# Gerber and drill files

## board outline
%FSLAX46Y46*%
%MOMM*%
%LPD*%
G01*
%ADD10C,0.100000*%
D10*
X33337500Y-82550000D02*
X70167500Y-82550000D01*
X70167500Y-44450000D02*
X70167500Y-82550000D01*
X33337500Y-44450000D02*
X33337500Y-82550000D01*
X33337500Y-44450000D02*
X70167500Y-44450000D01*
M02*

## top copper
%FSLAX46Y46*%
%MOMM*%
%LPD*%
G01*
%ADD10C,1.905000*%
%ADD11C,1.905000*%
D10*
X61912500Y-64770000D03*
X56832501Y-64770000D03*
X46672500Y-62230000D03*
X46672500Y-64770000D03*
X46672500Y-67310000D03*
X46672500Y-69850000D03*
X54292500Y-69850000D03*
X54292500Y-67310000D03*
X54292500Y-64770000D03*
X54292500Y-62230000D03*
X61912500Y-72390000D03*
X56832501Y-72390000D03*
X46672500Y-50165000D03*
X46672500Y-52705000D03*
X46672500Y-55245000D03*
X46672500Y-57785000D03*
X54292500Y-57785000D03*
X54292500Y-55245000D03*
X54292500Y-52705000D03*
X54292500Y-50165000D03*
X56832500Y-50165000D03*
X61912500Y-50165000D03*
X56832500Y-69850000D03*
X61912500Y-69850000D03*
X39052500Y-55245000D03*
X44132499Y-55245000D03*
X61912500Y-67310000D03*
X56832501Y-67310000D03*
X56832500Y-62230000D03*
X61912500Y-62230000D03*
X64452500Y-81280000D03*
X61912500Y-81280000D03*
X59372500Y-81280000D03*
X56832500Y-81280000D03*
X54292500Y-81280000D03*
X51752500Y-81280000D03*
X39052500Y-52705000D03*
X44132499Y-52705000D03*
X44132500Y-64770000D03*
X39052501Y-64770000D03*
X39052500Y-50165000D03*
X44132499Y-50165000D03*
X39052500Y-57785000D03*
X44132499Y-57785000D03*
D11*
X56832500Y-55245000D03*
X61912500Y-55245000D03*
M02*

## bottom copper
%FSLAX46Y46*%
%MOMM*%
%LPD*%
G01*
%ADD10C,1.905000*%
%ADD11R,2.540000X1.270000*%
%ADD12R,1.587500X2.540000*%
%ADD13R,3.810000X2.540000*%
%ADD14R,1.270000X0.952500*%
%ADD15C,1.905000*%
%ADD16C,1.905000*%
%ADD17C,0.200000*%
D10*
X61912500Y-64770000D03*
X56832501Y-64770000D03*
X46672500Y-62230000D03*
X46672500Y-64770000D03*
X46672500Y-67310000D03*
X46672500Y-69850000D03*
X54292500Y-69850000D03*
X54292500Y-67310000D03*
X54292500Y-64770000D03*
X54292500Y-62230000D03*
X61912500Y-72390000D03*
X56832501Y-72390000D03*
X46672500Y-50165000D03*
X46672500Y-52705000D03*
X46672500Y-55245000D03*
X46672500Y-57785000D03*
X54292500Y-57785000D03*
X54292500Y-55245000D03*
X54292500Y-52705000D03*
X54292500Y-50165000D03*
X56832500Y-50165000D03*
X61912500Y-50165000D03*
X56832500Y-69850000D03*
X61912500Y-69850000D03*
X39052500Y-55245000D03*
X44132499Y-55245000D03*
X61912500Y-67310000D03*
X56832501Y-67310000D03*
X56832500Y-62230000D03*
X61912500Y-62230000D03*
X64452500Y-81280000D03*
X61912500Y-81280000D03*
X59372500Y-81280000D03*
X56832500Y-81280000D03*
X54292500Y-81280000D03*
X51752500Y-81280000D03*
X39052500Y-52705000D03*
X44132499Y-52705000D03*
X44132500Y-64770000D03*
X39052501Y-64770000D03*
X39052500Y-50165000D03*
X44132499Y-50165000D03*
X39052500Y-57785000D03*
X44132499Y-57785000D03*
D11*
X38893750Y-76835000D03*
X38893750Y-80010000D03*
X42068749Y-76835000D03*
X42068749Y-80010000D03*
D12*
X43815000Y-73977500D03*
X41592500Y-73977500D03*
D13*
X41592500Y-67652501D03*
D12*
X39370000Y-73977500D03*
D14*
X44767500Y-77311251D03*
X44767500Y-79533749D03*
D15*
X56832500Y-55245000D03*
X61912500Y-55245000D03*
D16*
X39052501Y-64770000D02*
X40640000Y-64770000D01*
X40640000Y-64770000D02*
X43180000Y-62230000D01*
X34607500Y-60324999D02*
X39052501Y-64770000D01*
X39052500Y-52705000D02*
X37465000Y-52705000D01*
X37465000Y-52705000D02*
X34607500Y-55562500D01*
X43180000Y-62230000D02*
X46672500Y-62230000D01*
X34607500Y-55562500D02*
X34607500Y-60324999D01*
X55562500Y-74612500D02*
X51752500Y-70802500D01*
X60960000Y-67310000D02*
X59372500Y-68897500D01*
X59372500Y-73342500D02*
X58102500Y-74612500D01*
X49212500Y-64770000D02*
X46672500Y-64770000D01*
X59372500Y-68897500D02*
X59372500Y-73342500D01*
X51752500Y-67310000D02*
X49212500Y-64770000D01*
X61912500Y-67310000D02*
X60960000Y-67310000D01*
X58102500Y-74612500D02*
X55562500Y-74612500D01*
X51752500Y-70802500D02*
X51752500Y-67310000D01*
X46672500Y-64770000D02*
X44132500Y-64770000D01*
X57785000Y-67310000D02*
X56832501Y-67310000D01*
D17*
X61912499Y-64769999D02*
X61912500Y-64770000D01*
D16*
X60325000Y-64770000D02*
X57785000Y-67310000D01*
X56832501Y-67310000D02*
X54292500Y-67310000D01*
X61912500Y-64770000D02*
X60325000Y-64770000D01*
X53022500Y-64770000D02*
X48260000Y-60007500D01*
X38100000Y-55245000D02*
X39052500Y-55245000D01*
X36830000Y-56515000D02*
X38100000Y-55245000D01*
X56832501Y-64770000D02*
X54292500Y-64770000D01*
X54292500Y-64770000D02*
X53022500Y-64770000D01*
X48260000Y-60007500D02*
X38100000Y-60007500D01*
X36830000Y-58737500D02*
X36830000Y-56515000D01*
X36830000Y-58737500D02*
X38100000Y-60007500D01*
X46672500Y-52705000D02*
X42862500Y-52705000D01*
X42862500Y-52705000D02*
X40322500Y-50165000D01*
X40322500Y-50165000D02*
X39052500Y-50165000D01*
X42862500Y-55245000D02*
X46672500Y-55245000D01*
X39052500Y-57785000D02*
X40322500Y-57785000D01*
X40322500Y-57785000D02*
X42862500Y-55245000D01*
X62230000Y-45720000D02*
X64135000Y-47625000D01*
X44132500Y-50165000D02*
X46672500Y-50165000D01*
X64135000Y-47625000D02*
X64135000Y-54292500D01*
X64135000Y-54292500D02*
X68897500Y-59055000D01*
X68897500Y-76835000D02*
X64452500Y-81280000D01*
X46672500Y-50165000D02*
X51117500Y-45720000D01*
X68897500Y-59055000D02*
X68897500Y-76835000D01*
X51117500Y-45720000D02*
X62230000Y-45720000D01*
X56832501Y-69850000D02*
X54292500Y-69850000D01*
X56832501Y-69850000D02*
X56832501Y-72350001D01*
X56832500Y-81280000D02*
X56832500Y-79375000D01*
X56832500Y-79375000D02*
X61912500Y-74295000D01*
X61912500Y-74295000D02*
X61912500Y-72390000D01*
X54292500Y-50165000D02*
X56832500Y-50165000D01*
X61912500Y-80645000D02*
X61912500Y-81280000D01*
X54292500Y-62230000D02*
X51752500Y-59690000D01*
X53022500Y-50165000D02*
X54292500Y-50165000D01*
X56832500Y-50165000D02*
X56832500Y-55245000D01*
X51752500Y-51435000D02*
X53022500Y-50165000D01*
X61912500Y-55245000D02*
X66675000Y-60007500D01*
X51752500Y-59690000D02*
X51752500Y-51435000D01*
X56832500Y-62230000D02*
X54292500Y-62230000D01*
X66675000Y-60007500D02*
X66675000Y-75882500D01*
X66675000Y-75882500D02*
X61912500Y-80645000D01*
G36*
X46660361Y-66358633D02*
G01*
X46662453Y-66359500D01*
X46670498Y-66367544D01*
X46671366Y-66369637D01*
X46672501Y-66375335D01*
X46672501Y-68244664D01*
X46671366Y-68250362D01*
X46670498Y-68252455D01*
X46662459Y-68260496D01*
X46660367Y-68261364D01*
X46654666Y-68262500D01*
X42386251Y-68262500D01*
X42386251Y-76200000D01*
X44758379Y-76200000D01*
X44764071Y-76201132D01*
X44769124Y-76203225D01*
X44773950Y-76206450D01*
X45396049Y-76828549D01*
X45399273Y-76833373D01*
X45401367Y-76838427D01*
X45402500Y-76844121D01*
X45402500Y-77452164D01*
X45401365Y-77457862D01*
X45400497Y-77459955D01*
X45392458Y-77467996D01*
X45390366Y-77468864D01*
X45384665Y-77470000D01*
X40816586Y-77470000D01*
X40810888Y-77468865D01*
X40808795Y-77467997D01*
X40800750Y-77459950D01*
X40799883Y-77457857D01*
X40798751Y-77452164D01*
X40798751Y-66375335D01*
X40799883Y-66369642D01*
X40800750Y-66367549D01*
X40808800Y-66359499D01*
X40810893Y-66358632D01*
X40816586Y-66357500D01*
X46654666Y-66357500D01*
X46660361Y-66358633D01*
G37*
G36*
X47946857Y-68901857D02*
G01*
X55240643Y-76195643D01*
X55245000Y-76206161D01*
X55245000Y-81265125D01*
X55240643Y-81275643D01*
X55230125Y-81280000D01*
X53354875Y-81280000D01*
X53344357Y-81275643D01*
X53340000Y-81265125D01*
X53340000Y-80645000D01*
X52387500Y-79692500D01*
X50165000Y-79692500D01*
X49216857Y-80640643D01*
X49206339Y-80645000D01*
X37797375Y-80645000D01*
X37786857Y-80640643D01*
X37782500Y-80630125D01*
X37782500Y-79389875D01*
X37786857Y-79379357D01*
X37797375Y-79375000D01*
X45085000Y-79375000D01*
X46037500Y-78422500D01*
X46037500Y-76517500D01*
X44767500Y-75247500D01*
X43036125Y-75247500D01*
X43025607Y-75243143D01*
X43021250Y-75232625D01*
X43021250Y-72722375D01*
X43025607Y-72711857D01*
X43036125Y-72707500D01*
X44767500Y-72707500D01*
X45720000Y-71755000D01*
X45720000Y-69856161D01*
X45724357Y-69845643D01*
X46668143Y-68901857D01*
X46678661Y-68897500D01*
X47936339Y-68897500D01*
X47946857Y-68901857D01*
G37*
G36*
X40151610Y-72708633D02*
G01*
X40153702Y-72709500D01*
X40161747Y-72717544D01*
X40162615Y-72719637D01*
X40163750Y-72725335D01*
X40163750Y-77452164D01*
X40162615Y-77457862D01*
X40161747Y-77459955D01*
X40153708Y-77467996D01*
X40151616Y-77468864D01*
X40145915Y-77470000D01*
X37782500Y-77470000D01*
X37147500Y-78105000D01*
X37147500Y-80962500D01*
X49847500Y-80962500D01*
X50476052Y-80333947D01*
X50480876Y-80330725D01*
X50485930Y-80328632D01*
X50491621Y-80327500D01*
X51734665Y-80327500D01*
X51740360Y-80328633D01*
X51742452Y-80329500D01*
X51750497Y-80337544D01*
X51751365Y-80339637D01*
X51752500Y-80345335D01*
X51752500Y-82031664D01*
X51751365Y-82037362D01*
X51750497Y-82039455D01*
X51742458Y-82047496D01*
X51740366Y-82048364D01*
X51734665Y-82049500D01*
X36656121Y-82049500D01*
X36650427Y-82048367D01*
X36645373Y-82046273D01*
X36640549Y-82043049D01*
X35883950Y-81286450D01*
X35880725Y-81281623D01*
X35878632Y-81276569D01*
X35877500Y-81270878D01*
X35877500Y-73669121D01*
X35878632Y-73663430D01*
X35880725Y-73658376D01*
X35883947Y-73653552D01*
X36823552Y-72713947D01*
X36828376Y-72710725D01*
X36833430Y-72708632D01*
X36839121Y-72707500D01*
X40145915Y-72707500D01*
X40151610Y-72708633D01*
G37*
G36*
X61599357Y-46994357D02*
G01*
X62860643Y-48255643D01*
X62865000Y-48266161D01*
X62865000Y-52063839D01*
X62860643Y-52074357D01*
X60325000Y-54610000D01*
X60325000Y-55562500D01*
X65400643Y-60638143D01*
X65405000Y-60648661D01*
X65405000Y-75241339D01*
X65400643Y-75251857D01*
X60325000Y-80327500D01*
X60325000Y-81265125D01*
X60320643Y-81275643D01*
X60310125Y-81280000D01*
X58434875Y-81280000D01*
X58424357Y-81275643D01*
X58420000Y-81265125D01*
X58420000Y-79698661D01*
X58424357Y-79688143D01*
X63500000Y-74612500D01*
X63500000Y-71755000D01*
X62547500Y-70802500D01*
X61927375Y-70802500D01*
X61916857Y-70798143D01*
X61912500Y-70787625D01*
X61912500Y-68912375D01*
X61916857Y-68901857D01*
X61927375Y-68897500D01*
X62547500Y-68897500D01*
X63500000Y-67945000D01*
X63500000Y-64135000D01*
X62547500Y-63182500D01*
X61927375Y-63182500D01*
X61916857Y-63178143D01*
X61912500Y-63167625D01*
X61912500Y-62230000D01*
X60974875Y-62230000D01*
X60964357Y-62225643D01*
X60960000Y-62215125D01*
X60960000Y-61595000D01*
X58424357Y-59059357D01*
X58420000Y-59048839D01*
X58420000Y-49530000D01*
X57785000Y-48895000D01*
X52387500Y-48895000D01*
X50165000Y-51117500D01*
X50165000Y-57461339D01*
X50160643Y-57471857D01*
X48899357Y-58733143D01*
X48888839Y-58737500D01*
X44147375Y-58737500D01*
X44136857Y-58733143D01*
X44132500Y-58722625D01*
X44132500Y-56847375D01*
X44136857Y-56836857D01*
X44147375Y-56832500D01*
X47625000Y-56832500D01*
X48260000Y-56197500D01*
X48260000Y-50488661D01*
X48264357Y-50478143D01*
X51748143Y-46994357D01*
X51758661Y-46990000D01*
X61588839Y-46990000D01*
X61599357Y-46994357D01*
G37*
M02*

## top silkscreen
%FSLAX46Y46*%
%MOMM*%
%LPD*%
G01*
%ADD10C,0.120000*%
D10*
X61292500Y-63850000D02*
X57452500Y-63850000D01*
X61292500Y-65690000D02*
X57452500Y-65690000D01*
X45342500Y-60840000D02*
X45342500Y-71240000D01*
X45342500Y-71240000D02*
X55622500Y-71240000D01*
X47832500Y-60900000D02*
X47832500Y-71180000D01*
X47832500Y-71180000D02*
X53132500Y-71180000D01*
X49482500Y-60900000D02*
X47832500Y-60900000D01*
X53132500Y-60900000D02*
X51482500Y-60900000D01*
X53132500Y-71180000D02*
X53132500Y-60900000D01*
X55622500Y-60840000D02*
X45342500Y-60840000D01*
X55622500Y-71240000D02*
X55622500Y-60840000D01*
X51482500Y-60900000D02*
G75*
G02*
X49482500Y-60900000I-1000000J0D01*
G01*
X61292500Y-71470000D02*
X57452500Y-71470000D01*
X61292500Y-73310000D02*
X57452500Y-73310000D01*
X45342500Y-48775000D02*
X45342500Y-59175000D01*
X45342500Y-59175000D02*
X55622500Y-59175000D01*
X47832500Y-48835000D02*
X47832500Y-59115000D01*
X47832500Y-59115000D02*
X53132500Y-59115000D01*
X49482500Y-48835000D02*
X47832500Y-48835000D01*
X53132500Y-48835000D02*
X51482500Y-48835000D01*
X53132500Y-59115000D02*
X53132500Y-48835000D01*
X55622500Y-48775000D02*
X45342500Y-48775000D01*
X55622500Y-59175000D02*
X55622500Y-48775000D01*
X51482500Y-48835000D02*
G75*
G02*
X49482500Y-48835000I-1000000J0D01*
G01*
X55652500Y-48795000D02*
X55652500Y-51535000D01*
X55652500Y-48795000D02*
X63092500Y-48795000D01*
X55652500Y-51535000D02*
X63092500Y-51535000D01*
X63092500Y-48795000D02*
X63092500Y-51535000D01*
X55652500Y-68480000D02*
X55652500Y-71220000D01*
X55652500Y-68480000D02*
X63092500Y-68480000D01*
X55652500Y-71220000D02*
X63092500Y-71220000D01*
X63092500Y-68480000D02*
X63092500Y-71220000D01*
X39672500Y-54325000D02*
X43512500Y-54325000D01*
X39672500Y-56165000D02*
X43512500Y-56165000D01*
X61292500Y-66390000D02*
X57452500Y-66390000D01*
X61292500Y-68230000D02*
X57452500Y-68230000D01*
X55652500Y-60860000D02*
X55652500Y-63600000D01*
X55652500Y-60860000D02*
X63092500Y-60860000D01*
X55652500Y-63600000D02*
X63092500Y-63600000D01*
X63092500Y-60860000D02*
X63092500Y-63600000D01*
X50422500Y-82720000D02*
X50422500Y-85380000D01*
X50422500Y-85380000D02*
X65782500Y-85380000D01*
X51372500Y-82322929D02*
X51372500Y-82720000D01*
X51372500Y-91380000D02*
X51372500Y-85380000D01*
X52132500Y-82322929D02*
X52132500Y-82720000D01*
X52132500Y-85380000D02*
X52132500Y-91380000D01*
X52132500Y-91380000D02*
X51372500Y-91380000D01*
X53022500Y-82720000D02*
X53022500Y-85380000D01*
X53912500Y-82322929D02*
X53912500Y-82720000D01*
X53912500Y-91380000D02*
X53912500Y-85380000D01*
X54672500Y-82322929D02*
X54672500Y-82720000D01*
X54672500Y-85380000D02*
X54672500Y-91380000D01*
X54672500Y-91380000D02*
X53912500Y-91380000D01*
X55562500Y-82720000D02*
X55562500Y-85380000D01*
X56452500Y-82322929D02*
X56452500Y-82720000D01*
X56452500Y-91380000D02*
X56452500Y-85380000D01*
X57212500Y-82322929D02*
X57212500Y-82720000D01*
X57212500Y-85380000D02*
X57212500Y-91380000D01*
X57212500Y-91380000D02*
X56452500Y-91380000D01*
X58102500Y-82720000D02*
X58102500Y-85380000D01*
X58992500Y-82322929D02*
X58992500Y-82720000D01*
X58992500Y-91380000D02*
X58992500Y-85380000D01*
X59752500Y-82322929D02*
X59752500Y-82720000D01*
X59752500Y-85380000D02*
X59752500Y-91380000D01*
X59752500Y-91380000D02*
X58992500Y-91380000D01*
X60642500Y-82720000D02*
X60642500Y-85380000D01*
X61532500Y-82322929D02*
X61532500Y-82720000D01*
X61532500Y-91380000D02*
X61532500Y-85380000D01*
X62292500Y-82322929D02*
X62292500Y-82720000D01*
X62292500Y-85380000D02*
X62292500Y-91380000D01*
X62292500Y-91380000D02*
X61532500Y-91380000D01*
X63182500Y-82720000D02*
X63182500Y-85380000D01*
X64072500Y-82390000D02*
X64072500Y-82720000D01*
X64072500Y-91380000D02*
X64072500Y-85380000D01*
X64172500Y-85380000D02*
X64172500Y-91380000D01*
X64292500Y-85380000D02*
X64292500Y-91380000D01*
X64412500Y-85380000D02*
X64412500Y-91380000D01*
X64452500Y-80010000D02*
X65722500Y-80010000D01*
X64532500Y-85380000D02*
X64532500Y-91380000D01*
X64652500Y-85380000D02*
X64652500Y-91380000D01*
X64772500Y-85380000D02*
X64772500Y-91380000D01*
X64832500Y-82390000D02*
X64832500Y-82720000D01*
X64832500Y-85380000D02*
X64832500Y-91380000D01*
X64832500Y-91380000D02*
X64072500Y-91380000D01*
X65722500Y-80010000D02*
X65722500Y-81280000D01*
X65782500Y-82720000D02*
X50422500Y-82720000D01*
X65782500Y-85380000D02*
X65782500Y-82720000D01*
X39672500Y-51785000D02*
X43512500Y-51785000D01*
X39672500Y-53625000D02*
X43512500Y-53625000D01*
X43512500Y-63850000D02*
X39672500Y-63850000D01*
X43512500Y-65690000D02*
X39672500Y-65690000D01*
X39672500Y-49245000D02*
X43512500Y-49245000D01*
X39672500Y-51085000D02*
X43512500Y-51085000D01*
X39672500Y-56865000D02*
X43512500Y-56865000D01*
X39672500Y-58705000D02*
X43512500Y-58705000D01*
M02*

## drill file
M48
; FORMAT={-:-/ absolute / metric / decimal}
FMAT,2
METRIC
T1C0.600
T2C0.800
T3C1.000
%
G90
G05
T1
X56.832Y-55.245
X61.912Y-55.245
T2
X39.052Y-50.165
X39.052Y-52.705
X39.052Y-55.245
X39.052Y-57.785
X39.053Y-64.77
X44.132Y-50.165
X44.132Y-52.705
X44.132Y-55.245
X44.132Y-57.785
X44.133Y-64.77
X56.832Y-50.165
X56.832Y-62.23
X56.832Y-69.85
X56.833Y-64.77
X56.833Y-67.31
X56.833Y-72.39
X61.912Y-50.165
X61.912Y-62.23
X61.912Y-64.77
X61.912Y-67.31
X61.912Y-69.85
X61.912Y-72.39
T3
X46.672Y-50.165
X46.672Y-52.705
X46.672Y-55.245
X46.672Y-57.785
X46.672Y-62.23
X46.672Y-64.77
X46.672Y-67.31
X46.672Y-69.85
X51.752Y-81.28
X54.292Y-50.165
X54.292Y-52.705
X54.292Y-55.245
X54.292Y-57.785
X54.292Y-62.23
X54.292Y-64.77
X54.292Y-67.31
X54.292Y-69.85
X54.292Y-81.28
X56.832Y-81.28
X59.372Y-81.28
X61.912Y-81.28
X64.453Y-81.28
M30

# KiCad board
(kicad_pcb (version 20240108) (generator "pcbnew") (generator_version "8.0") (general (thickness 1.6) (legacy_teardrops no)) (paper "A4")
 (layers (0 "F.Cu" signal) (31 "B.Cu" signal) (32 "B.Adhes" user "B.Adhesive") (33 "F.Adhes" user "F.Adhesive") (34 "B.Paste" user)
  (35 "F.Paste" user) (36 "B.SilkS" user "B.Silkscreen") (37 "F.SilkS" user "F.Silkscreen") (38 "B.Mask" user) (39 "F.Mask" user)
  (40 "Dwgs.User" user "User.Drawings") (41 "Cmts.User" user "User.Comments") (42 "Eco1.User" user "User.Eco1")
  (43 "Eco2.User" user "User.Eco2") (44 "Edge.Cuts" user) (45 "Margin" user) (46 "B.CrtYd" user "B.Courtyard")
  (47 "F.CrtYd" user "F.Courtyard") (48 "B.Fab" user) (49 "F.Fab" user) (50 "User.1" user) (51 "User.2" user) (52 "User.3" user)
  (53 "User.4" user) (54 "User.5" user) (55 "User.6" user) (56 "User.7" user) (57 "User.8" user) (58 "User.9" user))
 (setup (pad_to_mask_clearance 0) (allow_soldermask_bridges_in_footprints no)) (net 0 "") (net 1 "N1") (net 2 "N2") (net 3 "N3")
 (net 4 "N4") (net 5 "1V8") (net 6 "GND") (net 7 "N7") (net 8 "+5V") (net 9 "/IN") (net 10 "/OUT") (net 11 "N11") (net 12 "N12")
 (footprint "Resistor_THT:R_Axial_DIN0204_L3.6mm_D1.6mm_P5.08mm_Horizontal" (layer "F.Cu") (at 61.9125 64.77 180)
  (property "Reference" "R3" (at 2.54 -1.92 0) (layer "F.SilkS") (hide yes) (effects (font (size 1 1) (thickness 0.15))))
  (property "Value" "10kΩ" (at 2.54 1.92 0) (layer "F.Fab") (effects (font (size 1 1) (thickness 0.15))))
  (fp_line (start 0.62 0.92) (end 4.46 0.92) (stroke (width 0.12) (type solid)) (layer "F.SilkS"))
  (fp_line (start 0.62 -0.92) (end 4.46 -0.92) (stroke (width 0.12) (type solid)) (layer "F.SilkS"))
  (pad "1" thru_hole circle (at 0 0 180) (size 1.905 1.905) (drill 0.8) (layers "*.Cu" "*.Mask") (remove_unused_layers no) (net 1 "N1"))
  (pad "2" thru_hole circle (at 5.079999 0 180) (size 1.905 1.905) (drill 0.8) (layers "*.Cu" "*.Mask") (remove_unused_layers no)
   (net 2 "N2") (thermal_bridge_angle 90)))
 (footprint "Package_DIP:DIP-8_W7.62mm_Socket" (layer "F.Cu") (at 50.4825 66.04)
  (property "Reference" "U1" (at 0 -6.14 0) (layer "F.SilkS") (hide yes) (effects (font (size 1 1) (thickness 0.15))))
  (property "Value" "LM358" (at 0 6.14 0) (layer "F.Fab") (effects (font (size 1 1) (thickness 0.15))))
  (fp_line (start -5.14 -5.2) (end -5.14 5.2) (stroke (width 0.12) (type solid)) (layer "F.SilkS"))
  (fp_line (start -5.14 5.2) (end 5.14 5.2) (stroke (width 0.12) (type solid)) (layer "F.SilkS"))
  (fp_line (start -2.65 -5.14) (end -2.65 5.14) (stroke (width 0.12) (type solid)) (layer "F.SilkS"))
  (fp_line (start -2.65 5.14) (end 2.65 5.14) (stroke (width 0.12) (type solid)) (layer "F.SilkS"))
  (fp_line (start -1 -5.14) (end -2.65 -5.14) (stroke (width 0.12) (type solid)) (layer "F.SilkS"))
  (fp_line (start 2.65 -5.14) (end 1 -5.14) (stroke (width 0.12) (type solid)) (layer "F.SilkS"))
  (fp_line (start 2.65 5.14) (end 2.65 -5.14) (stroke (width 0.12) (type solid)) (layer "F.SilkS"))
  (fp_line (start 5.14 -5.2) (end -5.14 -5.2) (stroke (width 0.12) (type solid)) (layer "F.SilkS"))
  (fp_line (start 5.14 5.2) (end 5.14 -5.2) (stroke (width 0.12) (type solid)) (layer "F.SilkS"))
  (fp_arc (start 1 -5.14) (mid 0 -4.14) (end -1 -5.14) (stroke (width 0.12) (type solid)) (layer "F.SilkS"))
  (pad "1" thru_hole circle (at -3.81 -3.81) (size 1.905 1.905) (drill 1) (layers "*.Cu" "*.Mask") (remove_unused_layers no) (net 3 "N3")
   (thermal_bridge_angle 90))
  (pad "2" thru_hole circle (at -3.81 -1.27) (size 1.905 1.905) (drill 1) (layers "*.Cu" "*.Mask") (remove_unused_layers no) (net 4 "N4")
   (thermal_bridge_angle 90))
  (pad "3" thru_hole circle (at -3.81 1.27) (size 1.905 1.905) (drill 1) (layers "*.Cu" "*.Mask") (remove_unused_layers no) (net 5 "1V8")
   (thermal_bridge_angle 90))
  (pad "4" thru_hole circle (at -3.81 3.81) (size 1.905 1.905) (drill 1) (layers "*.Cu" "*.Mask") (remove_unused_layers no) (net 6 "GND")
   (thermal_bridge_angle 90))
  (pad "5" thru_hole circle (at 3.81 3.81) (size 1.905 1.905) (drill 1) (layers "*.Cu" "*.Mask") (remove_unused_layers no) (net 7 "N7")
   (thermal_bridge_angle 90))
  (pad "6" thru_hole circle (at 3.81 1.27) (size 1.905 1.905) (drill 1) (layers "*.Cu" "*.Mask") (remove_unused_layers no) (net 1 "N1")
   (thermal_bridge_angle 90))
  (pad "7" thru_hole circle (at 3.81 -1.27) (size 1.905 1.905) (drill 1) (layers "*.Cu" "*.Mask") (remove_unused_layers no) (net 2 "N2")
   (thermal_bridge_angle 90))
  (pad "8" thru_hole circle (at 3.81 -3.81) (size 1.905 1.905) (drill 1) (layers "*.Cu" "*.Mask") (remove_unused_layers no) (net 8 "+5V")
   (thermal_bridge_angle 90)))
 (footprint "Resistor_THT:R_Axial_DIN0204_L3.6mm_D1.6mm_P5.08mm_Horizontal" (layer "F.Cu") (at 61.9125 72.39 180)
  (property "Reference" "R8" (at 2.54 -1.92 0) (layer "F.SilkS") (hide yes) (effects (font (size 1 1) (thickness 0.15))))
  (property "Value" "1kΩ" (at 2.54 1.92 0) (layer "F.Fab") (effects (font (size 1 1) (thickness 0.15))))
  (fp_line (start 0.62 0.92) (end 4.46 0.92) (stroke (width 0.12) (type solid)) (layer "F.SilkS"))
  (fp_line (start 0.62 -0.92) (end 4.46 -0.92) (stroke (width 0.12) (type solid)) (layer "F.SilkS"))
  (pad "1" thru_hole circle (at 0 0 180) (size 1.905 1.905) (drill 0.8) (layers "*.Cu" "*.Mask") (remove_unused_layers no) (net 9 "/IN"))
  (pad "2" thru_hole circle (at 5.079999 0 180) (size 1.905 1.905) (drill 0.8) (layers "*.Cu" "*.Mask") (remove_unused_layers no)
   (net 7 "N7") (thermal_bridge_angle 90)))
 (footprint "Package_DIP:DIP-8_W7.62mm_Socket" (layer "F.Cu") (at 50.4825 53.975)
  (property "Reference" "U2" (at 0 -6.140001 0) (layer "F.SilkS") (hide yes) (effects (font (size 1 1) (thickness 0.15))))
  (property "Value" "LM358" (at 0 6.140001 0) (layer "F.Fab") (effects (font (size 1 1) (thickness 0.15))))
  (fp_line (start -5.14 -5.2) (end -5.14 5.2) (stroke (width 0.12) (type solid)) (layer "F.SilkS"))
  (fp_line (start -5.14 5.2) (end 5.14 5.2) (stroke (width 0.12) (type solid)) (layer "F.SilkS"))
  (fp_line (start -2.65 -5.14) (end -2.65 5.14) (stroke (width 0.12) (type solid)) (layer "F.SilkS"))
  (fp_line (start -2.65 5.14) (end 2.65 5.14) (stroke (width 0.12) (type solid)) (layer "F.SilkS"))
  (fp_line (start -1 -5.14) (end -2.65 -5.14) (stroke (width 0.12) (type solid)) (layer "F.SilkS"))
  (fp_line (start 2.65 -5.14) (end 1 -5.14) (stroke (width 0.12) (type solid)) (layer "F.SilkS"))
  (fp_line (start 2.65 5.14) (end 2.65 -5.14) (stroke (width 0.12) (type solid)) (layer "F.SilkS"))
  (fp_line (start 5.14 -5.2) (end -5.14 -5.2) (stroke (width 0.12) (type solid)) (layer "F.SilkS"))
  (fp_line (start 5.14 5.2) (end 5.14 -5.2) (stroke (width 0.12) (type solid)) (layer "F.SilkS"))
  (fp_arc (start 1 -5.14) (mid 0 -4.14) (end -1 -5.14) (stroke (width 0.12) (type solid)) (layer "F.SilkS"))
  (pad "1" thru_hole circle (at -3.81 -3.81) (size 1.905 1.905) (drill 1) (layers "*.Cu" "*.Mask") (remove_unused_layers no) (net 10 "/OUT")
   (thermal_bridge_angle 90))
  (pad "2" thru_hole circle (at -3.81 -1.27) (size 1.905 1.905) (drill 1) (layers "*.Cu" "*.Mask") (remove_unused_layers no) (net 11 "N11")
   (thermal_bridge_angle 90))
  (pad "3" thru_hole circle (at -3.81 1.27) (size 1.905 1.905) (drill 1) (layers "*.Cu" "*.Mask") (remove_unused_layers no) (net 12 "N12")
   (thermal_bridge_angle 90))
  (pad "4" thru_hole circle (at -3.81 3.81) (size 1.905 1.905) (drill 1) (layers "*.Cu" "*.Mask") (remove_unused_layers no) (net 6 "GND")
   (thermal_bridge_angle 90))
  (pad "5" thru_hole circle (at 3.81 3.81) (size 1.905 1.905) (drill 1) (layers "*.Cu" "*.Mask") (remove_unused_layers no)
   (thermal_bridge_angle 90))
  (pad "6" thru_hole circle (at 3.81 1.27) (size 1.905 1.905) (drill 1) (layers "*.Cu" "*.Mask") (remove_unused_layers no)
   (thermal_bridge_angle 90))
  (pad "7" thru_hole circle (at 3.81 -1.27) (size 1.905 1.905) (drill 1) (layers "*.Cu" "*.Mask") (remove_unused_layers no)
   (thermal_bridge_angle 90))
  (pad "8" thru_hole circle (at 3.81 -3.81) (size 1.905 1.905) (drill 1) (layers "*.Cu" "*.Mask") (remove_unused_layers no) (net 8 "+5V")
   (thermal_bridge_angle 90)))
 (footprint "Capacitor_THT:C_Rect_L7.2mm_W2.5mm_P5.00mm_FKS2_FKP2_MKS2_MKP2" (layer "F.Cu") (at 56.8725 50.165)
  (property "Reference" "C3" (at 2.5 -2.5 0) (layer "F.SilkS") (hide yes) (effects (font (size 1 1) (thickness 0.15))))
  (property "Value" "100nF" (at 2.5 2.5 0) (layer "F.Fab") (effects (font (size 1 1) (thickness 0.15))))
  (fp_line (start -1.22 -1.37) (end -1.22 1.37) (stroke (width 0.12) (type solid)) (layer "F.SilkS"))
  (fp_line (start -1.22 -1.37) (end 6.22 -1.37) (stroke (width 0.12) (type solid)) (layer "F.SilkS"))
  (fp_line (start -1.22 1.37) (end 6.22 1.37) (stroke (width 0.12) (type solid)) (layer "F.SilkS"))
  (fp_line (start 6.22 -1.37) (end 6.22 1.37) (stroke (width 0.12) (type solid)) (layer "F.SilkS"))
  (pad "1" thru_hole circle (at -0.04 0) (size 1.905 1.6) (drill 0.8) (layers "*.Cu" "*.Mask") (remove_unused_layers no) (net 8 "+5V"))
  (pad "2" thru_hole circle (at 5.04 0) (size 1.905 1.6) (drill 0.8) (layers "*.Cu" "*.Mask") (remove_unused_layers no) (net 6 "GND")))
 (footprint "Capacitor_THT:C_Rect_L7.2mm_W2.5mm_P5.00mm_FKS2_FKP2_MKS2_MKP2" (layer "F.Cu") (at 56.8725 69.85)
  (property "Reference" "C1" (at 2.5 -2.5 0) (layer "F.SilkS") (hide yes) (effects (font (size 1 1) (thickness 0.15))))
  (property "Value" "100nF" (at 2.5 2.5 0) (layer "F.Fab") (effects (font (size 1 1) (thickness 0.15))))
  (fp_line (start -1.22 -1.37) (end -1.22 1.37) (stroke (width 0.12) (type solid)) (layer "F.SilkS"))
  (fp_line (start -1.22 -1.37) (end 6.22 -1.37) (stroke (width 0.12) (type solid)) (layer "F.SilkS"))
  (fp_line (start -1.22 1.37) (end 6.22 1.37) (stroke (width 0.12) (type solid)) (layer "F.SilkS"))
  (fp_line (start 6.22 -1.37) (end 6.22 1.37) (stroke (width 0.12) (type solid)) (layer "F.SilkS"))
  (pad "1" thru_hole circle (at -0.04 0) (size 1.905 1.6) (drill 0.8) (layers "*.Cu" "*.Mask") (remove_unused_layers no) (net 7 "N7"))
  (pad "2" thru_hole circle (at 5.04 0) (size 1.905 1.6) (drill 0.8) (layers "*.Cu" "*.Mask") (remove_unused_layers no) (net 6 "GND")))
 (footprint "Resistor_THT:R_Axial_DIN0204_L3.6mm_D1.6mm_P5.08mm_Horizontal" (layer "F.Cu") (at 39.0525 55.245)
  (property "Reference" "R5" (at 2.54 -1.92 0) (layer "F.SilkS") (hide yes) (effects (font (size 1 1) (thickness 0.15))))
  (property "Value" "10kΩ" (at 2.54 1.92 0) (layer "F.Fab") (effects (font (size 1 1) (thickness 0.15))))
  (fp_line (start 0.62 -0.92) (end 4.46 -0.92) (stroke (width 0.12) (type solid)) (layer "F.SilkS"))
  (fp_line (start 0.62 0.92) (end 4.46 0.92) (stroke (width 0.12) (type solid)) (layer "F.SilkS"))
  (pad "1" thru_hole circle (at 0 0) (size 1.905 1.905) (drill 0.8) (layers "*.Cu" "*.Mask") (remove_unused_layers no) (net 2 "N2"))
  (pad "2" thru_hole circle (at 5.079999 0) (size 1.905 1.905) (drill 0.8) (layers "*.Cu" "*.Mask") (remove_unused_layers no) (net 12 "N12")
   (thermal_bridge_angle 90)))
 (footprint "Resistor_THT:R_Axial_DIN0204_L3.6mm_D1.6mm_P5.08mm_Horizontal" (layer "F.Cu") (at 61.9125 67.31 180)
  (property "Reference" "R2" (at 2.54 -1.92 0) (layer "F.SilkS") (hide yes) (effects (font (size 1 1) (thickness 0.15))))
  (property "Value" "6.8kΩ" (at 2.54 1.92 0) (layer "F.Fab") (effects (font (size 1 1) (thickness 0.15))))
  (fp_line (start 0.62 0.92) (end 4.46 0.92) (stroke (width 0.12) (type solid)) (layer "F.SilkS"))
  (fp_line (start 0.62 -0.92) (end 4.46 -0.92) (stroke (width 0.12) (type solid)) (layer "F.SilkS"))
  (pad "1" thru_hole circle (at 0 0 180) (size 1.905 1.905) (drill 0.8) (layers "*.Cu" "*.Mask") (remove_unused_layers no) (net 4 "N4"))
  (pad "2" thru_hole circle (at 5.079999 0 180) (size 1.905 1.905) (drill 0.8) (layers "*.Cu" "*.Mask") (remove_unused_layers no)
   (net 1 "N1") (thermal_bridge_angle 90)))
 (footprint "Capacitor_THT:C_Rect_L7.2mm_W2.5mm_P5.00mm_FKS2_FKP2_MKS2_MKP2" (layer "F.Cu") (at 56.8725 62.23)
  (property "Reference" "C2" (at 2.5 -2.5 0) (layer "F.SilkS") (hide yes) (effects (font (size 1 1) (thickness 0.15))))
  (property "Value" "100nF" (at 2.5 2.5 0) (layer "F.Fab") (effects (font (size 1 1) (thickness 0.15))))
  (fp_line (start -1.22 -1.37) (end -1.22 1.37) (stroke (width 0.12) (type solid)) (layer "F.SilkS"))
  (fp_line (start -1.22 -1.37) (end 6.22 -1.37) (stroke (width 0.12) (type solid)) (layer "F.SilkS"))
  (fp_line (start -1.22 1.37) (end 6.22 1.37) (stroke (width 0.12) (type solid)) (layer "F.SilkS"))
  (fp_line (start 6.22 -1.37) (end 6.22 1.37) (stroke (width 0.12) (type solid)) (layer "F.SilkS"))
  (pad "1" thru_hole circle (at -0.04 0) (size 1.905 1.6) (drill 0.8) (layers "*.Cu" "*.Mask") (remove_unused_layers no) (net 8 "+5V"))
  (pad "2" thru_hole circle (at 5.04 0) (size 1.905 1.6) (drill 0.8) (layers "*.Cu" "*.Mask") (remove_unused_layers no) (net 6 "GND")))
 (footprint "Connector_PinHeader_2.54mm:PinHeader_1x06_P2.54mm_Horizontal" (layer "F.Cu") (at 64.4525 81.28 -90)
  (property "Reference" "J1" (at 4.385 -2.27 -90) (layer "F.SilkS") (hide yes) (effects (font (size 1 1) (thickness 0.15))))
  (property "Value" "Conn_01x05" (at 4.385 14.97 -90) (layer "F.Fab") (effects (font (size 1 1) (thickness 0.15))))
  (fp_line (start 1.44 14.03) (end 4.1 14.03) (stroke (width 0.12) (type solid)) (layer "F.SilkS"))
  (fp_line (start 4.1 14.03) (end 4.1 -1.33) (stroke (width 0.12) (type solid)) (layer "F.SilkS"))
  (fp_line (start 1.042929 13.08) (end 1.44 13.08) (stroke (width 0.12) (type solid)) (layer "F.SilkS"))
  (fp_line (start 10.1 13.08) (end 4.1 13.08) (stroke (width 0.12) (type solid)) (layer "F.SilkS"))
  (fp_line (start 1.042929 12.32) (end 1.44 12.32) (stroke (width 0.12) (type solid)) (layer "F.SilkS"))
  (fp_line (start 4.1 12.32) (end 10.1 12.32) (stroke (width 0.12) (type solid)) (layer "F.SilkS"))
  (fp_line (start 10.1 12.32) (end 10.1 13.08) (stroke (width 0.12) (type solid)) (layer "F.SilkS"))
  (fp_line (start 1.44 11.43) (end 4.1 11.43) (stroke (width 0.12) (type solid)) (layer "F.SilkS"))
  (fp_line (start 1.042929 10.54) (end 1.44 10.54) (stroke (width 0.12) (type solid)) (layer "F.SilkS"))
  (fp_line (start 10.1 10.54) (end 4.1 10.54) (stroke (width 0.12) (type solid)) (layer "F.SilkS"))
  (fp_line (start 1.042929 9.78) (end 1.44 9.78) (stroke (width 0.12) (type solid)) (layer "F.SilkS"))
  (fp_line (start 4.1 9.78) (end 10.1 9.78) (stroke (width 0.12) (type solid)) (layer "F.SilkS"))
  (fp_line (start 10.1 9.78) (end 10.1 10.54) (stroke (width 0.12) (type solid)) (layer "F.SilkS"))
  (fp_line (start 1.44 8.89) (end 4.1 8.89) (stroke (width 0.12) (type solid)) (layer "F.SilkS"))
  (fp_line (start 1.042929 8) (end 1.44 8) (stroke (width 0.12) (type solid)) (layer "F.SilkS"))
  (fp_line (start 10.1 8) (end 4.1 8) (stroke (width 0.12) (type solid)) (layer "F.SilkS"))
  (fp_line (start 1.042929 7.24) (end 1.44 7.24) (stroke (width 0.12) (type solid)) (layer "F.SilkS"))
  (fp_line (start 4.1 7.24) (end 10.1 7.24) (stroke (width 0.12) (type solid)) (layer "F.SilkS"))
  (fp_line (start 10.1 7.24) (end 10.1 8) (stroke (width 0.12) (type solid)) (layer "F.SilkS"))
  (fp_line (start 1.44 6.35) (end 4.1 6.35) (stroke (width 0.12) (type solid)) (layer "F.SilkS"))
  (fp_line (start 1.042929 5.46) (end 1.44 5.46) (stroke (width 0.12) (type solid)) (layer "F.SilkS"))
  (fp_line (start 10.1 5.46) (end 4.1 5.46) (stroke (width 0.12) (type solid)) (layer "F.SilkS"))
  (fp_line (start 1.042929 4.7) (end 1.44 4.7) (stroke (width 0.12) (type solid)) (layer "F.SilkS"))
  (fp_line (start 4.1 4.7) (end 10.1 4.7) (stroke (width 0.12) (type solid)) (layer "F.SilkS"))
  (fp_line (start 10.1 4.7) (end 10.1 5.46) (stroke (width 0.12) (type solid)) (layer "F.SilkS"))
  (fp_line (start 1.44 3.81) (end 4.1 3.81) (stroke (width 0.12) (type solid)) (layer "F.SilkS"))
  (fp_line (start 1.042929 2.92) (end 1.44 2.92) (stroke (width 0.12) (type solid)) (layer "F.SilkS"))
  (fp_line (start 10.1 2.92) (end 4.1 2.92) (stroke (width 0.12) (type solid)) (layer "F.SilkS"))
  (fp_line (start 1.042929 2.16) (end 1.44 2.16) (stroke (width 0.12) (type solid)) (layer "F.SilkS"))
  (fp_line (start 4.1 2.16) (end 10.1 2.16) (stroke (width 0.12) (type solid)) (layer "F.SilkS"))
  (fp_line (start 10.1 2.16) (end 10.1 2.92) (stroke (width 0.12) (type solid)) (layer "F.SilkS"))
  (fp_line (start 1.44 1.27) (end 4.1 1.27) (stroke (width 0.12) (type solid)) (layer "F.SilkS"))
  (fp_line (start 1.11 0.38) (end 1.44 0.38) (stroke (width 0.12) (type solid)) (layer "F.SilkS"))
  (fp_line (start 10.1 0.38) (end 4.1 0.38) (stroke (width 0.12) (type solid)) (layer "F.SilkS"))
  (fp_line (start 4.1 0.28) (end 10.1 0.28) (stroke (width 0.12) (type solid)) (layer "F.SilkS"))
  (fp_line (start 4.1 0.16) (end 10.1 0.16) (stroke (width 0.12) (type solid)) (layer "F.SilkS"))
  (fp_line (start 4.1 0.04) (end 10.1 0.04) (stroke (width 0.12) (type solid)) (layer "F.SilkS"))
  (fp_line (start -1.27 0) (end -1.27 -1.27) (stroke (width 0.12) (type solid)) (layer "F.SilkS"))
  (fp_line (start 4.1 -0.08) (end 10.1 -0.08) (stroke (width 0.12) (type solid)) (layer "F.SilkS"))
  (fp_line (start 4.1 -0.2) (end 10.1 -0.2) (stroke (width 0.12) (type solid)) (layer "F.SilkS"))
  (fp_line (start 4.1 -0.32) (end 10.1 -0.32) (stroke (width 0.12) (type solid)) (layer "F.SilkS"))
  (fp_line (start 1.11 -0.38) (end 1.44 -0.38) (stroke (width 0.12) (type solid)) (layer "F.SilkS"))
  (fp_line (start 4.1 -0.38) (end 10.1 -0.38) (stroke (width 0.12) (type solid)) (layer "F.SilkS"))
  (fp_line (start 10.1 -0.38) (end 10.1 0.38) (stroke (width 0.12) (type solid)) (layer "F.SilkS"))
  (fp_line (start -1.27 -1.27) (end 0 -1.27) (stroke (width 0.12) (type solid)) (layer "F.SilkS"))
  (fp_line (start 1.44 -1.33) (end 1.44 14.03) (stroke (width 0.12) (type solid)) (layer "F.SilkS"))
  (fp_line (start 4.1 -1.33) (end 1.44 -1.33) (stroke (width 0.12) (type solid)) (layer "F.SilkS"))
  (pad "1" thru_hole circle (at 0 0 270) (size 1.905 1.905) (drill 1) (layers "*.Cu" "*.Mask") (remove_unused_layers no) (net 10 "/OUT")
   (thermal_bridge_angle 90))
  (pad "2" thru_hole circle (at 0 2.54 270) (size 1.905 1.905) (drill 1) (layers "*.Cu" "*.Mask") (remove_unused_layers no) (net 8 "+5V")
   (thermal_bridge_angle 90))
  (pad "3" thru_hole circle (at 0 5.08 270) (size 1.905 1.905) (drill 1) (layers "*.Cu" "*.Mask") (remove_unused_layers no) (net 6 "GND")
   (thermal_bridge_angle 90))
  (pad "4" thru_hole circle (at 0 7.62 270) (size 1.905 1.905) (drill 1) (layers "*.Cu" "*.Mask") (remove_unused_layers no) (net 9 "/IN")
   (thermal_bridge_angle 90))
  (pad "5" thru_hole circle (at 0 10.16 270) (size 1.905 1.905) (drill 1) (layers "*.Cu" "*.Mask") (remove_unused_layers no) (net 6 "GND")
   (thermal_bridge_angle 90))
  (pad "6" thru_hole circle (at 0 12.7 270) (size 1.905 1.905) (drill 1) (layers "*.Cu" "*.Mask") (remove_unused_layers no) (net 8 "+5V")
   (thermal_bridge_angle 90)))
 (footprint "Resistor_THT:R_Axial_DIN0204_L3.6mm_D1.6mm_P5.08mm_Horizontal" (layer "F.Cu") (at 39.0525 52.705)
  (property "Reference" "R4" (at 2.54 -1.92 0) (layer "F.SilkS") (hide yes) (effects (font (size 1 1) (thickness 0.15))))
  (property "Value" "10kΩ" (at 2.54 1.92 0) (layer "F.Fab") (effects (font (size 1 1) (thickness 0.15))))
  (fp_line (start 0.62 -0.92) (end 4.46 -0.92) (stroke (width 0.12) (type solid)) (layer "F.SilkS"))
  (fp_line (start 0.62 0.92) (end 4.46 0.92) (stroke (width 0.12) (type solid)) (layer "F.SilkS"))
  (pad "1" thru_hole circle (at 0 0) (size 1.905 1.905) (drill 0.8) (layers "*.Cu" "*.Mask") (remove_unused_layers no) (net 3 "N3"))
  (pad "2" thru_hole circle (at 5.079999 0) (size 1.905 1.905) (drill 0.8) (layers "*.Cu" "*.Mask") (remove_unused_layers no) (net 11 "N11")
   (thermal_bridge_angle 90)))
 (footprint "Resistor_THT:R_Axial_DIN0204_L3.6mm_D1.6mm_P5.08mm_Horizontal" (layer "F.Cu") (at 44.1325 64.77 180)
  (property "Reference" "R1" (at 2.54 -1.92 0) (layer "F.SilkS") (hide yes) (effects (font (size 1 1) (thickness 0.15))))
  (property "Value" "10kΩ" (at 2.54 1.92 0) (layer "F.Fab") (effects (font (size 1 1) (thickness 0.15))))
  (fp_line (start 0.62 0.92) (end 4.46 0.92) (stroke (width 0.12) (type solid)) (layer "F.SilkS"))
  (fp_line (start 0.62 -0.92) (end 4.46 -0.92) (stroke (width 0.12) (type solid)) (layer "F.SilkS"))
  (pad "1" thru_hole circle (at 0 0 180) (size 1.905 1.905) (drill 0.8) (layers "*.Cu" "*.Mask") (remove_unused_layers no) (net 4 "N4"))
  (pad "2" thru_hole circle (at 5.079999 0 180) (size 1.905 1.905) (drill 0.8) (layers "*.Cu" "*.Mask") (remove_unused_layers no)
   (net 3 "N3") (thermal_bridge_angle 90)))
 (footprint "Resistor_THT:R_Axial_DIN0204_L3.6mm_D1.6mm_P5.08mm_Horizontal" (layer "F.Cu") (at 39.0525 50.165)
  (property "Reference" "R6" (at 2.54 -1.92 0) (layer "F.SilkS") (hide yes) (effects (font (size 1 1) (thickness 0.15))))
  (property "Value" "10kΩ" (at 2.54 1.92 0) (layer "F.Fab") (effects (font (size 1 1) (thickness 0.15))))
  (fp_line (start 0.62 -0.92) (end 4.46 -0.92) (stroke (width 0.12) (type solid)) (layer "F.SilkS"))
  (fp_line (start 0.62 0.92) (end 4.46 0.92) (stroke (width 0.12) (type solid)) (layer "F.SilkS"))
  (pad "1" thru_hole circle (at 0 0) (size 1.905 1.905) (drill 0.8) (layers "*.Cu" "*.Mask") (remove_unused_layers no) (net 11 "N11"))
  (pad "2" thru_hole circle (at 5.079999 0) (size 1.905 1.905) (drill 0.8) (layers "*.Cu" "*.Mask") (remove_unused_layers no)
   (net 10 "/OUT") (thermal_bridge_angle 90)))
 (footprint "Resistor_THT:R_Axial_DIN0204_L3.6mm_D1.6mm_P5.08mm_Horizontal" (layer "F.Cu") (at 39.0525 57.785)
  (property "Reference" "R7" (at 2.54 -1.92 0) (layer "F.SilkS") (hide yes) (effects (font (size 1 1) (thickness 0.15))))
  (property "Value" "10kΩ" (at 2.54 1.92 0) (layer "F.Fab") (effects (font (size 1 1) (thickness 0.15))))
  (fp_line (start 0.62 -0.92) (end 4.46 -0.92) (stroke (width 0.12) (type solid)) (layer "F.SilkS"))
  (fp_line (start 0.62 0.92) (end 4.46 0.92) (stroke (width 0.12) (type solid)) (layer "F.SilkS"))
  (pad "1" thru_hole circle (at 0 0) (size 1.905 1.905) (drill 0.8) (layers "*.Cu" "*.Mask") (remove_unused_layers no) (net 12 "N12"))
  (pad "2" thru_hole circle (at 5.079999 0) (size 1.905 1.905) (drill 0.8) (layers "*.Cu" "*.Mask") (remove_unused_layers no) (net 6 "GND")
   (thermal_bridge_angle 90)))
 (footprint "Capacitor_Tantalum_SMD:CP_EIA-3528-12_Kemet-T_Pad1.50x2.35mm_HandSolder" (layer "B.Cu") (at 38.89375 78.4225 -90)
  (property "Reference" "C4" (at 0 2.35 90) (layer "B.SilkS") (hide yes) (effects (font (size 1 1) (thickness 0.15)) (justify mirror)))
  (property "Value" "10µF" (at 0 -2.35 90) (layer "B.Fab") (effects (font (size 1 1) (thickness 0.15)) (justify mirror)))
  (pad "1" smd rect (at -1.5875 0 270) (size 1.27 2.54) (layers "B.Cu" "B.Paste" "B.Mask") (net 8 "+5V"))
  (pad "2" smd rect (at 1.5875 0 270) (size 1.27 2.54) (layers "B.Cu" "B.Paste" "B.Mask") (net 6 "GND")))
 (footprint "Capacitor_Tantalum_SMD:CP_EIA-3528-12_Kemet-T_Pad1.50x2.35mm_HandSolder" (layer "B.Cu") (at 42.068749 78.4225 -90)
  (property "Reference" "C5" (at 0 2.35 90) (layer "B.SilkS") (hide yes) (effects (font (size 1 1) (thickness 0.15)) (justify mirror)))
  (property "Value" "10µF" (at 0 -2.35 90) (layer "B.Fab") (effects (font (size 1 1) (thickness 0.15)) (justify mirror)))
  (pad "1" smd rect (at -1.5875 0 270) (size 1.27 2.54) (layers "B.Cu" "B.Paste" "B.Mask") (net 5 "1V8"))
  (pad "2" smd rect (at 1.5875 0 270) (size 1.27 2.54) (layers "B.Cu" "B.Paste" "B.Mask") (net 6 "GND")))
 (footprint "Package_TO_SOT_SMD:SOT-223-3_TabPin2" (layer "B.Cu") (at 41.5925 70.8025 90)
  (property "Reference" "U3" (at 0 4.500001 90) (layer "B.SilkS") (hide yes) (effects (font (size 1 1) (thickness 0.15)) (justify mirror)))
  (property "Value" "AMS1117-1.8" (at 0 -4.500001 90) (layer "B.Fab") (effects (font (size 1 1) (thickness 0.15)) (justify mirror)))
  (pad "1" smd rect (at -3.175 2.2225 90) (size 2.54 1.5875) (layers "B.Cu" "B.Paste" "B.Mask") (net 6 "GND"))
  (pad "2" smd rect (at -3.175 0 90) (size 2.54 1.5875) (layers "B.Cu" "B.Paste" "B.Mask") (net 5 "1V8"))
  (pad "2" smd rect (at 3.149999 0 90) (size 2.54 3.81) (layers "B.Cu" "B.Paste" "B.Mask") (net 5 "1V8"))
  (pad "3" smd rect (at -3.175 -2.2225 90) (size 2.54 1.5875) (layers "B.Cu" "B.Paste" "B.Mask") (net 8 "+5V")))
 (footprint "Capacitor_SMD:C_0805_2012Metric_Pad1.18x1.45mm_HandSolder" (layer "B.Cu") (at 44.7675 78.4225 -90)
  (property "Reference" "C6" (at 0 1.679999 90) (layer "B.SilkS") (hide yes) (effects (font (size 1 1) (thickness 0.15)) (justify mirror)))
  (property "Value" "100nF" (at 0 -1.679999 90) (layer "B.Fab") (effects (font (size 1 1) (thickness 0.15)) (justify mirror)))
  (pad "1" smd rect (at -1.111249 0 270) (size 0.9525 1.27) (layers "B.Cu" "B.Paste" "B.Mask") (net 5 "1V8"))
  (pad "2" smd rect (at 1.111249 0 270) (size 0.9525 1.27) (layers "B.Cu" "B.Paste" "B.Mask") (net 6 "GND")))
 (gr_line (start 33.3375 82.55) (end 70.1675 82.55) (stroke (width 0) (type default)) (layer "Edge.Cuts"))
 (gr_line (start 70.1675 44.45) (end 70.1675 82.55) (stroke (width 0) (type default)) (layer "Edge.Cuts"))
 (gr_line (start 33.3375 44.45) (end 33.3375 82.55) (stroke (width 0) (type default)) (layer "Edge.Cuts"))
 (gr_line (start 33.3375 44.45) (end 70.1675 44.45) (stroke (width 0) (type default)) (layer "Edge.Cuts"))
 (segment (start 39.052501 64.77) (end 40.64 64.77) (width 1.905) (layer "B.Cu") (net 3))
 (segment (start 40.64 64.77) (end 43.18 62.23) (width 1.905) (layer "B.Cu") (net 3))
 (segment (start 34.6075 60.324999) (end 39.052501 64.77) (width 1.905) (layer "B.Cu") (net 3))
 (segment (start 39.0525 52.705) (end 37.465 52.705) (width 1.905) (layer "B.Cu") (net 3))
 (segment (start 37.465 52.705) (end 34.6075 55.5625) (width 1.905) (layer "B.Cu") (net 3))
 (segment (start 43.18 62.23) (end 46.6725 62.23) (width 1.905) (layer "B.Cu") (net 3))
 (segment (start 34.6075 55.5625) (end 34.6075 60.324999) (width 1.905) (layer "B.Cu") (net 3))
 (segment (start 55.5625 74.6125) (end 51.7525 70.8025) (width 1.905) (layer "B.Cu") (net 4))
 (segment (start 60.96 67.31) (end 59.3725 68.8975) (width 1.905) (layer "B.Cu") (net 4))
 (segment (start 59.3725 73.3425) (end 58.1025 74.6125) (width 1.905) (layer "B.Cu") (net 4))
 (segment (start 49.2125 64.77) (end 46.6725 64.77) (width 1.905) (layer "B.Cu") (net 4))
 (segment (start 59.3725 68.8975) (end 59.3725 73.3425) (width 1.905) (layer "B.Cu") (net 4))
 (segment (start 51.7525 67.31) (end 49.2125 64.77) (width 1.905) (layer "B.Cu") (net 4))
 (segment (start 61.9125 67.31) (end 60.96 67.31) (width 1.905) (layer "B.Cu") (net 4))
 (segment (start 58.1025 74.6125) (end 55.5625 74.6125) (width 1.905) (layer "B.Cu") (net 4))
 (segment (start 51.7525 70.8025) (end 51.7525 67.31) (width 1.905) (layer "B.Cu") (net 4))
 (segment (start 46.6725 64.77) (end 44.1325 64.77) (width 1.905) (layer "B.Cu") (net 4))
 (segment (start 57.785 67.31) (end 56.832501 67.31) (width 1.905) (layer "B.Cu") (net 1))
 (segment (start 61.912499 64.769999) (end 61.9125 64.77) (width 0.2) (layer "B.Cu") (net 1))
 (segment (start 60.325 64.77) (end 57.785 67.31) (width 1.905) (layer "B.Cu") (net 1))
 (segment (start 56.832501 67.31) (end 54.2925 67.31) (width 1.905) (layer "B.Cu") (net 1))
 (segment (start 61.9125 64.77) (end 60.325 64.77) (width 1.905) (layer "B.Cu") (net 1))
 (segment (start 53.0225 64.77) (end 48.26 60.0075) (width 1.905) (layer "B.Cu") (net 2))
 (segment (start 38.1 55.245) (end 39.0525 55.245) (width 1.905) (layer "B.Cu") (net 2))
 (segment (start 36.83 56.515) (end 38.1 55.245) (width 1.905) (layer "B.Cu") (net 2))
 (segment (start 56.832501 64.77) (end 54.2925 64.77) (width 1.905) (layer "B.Cu") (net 2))
 (segment (start 54.2925 64.77) (end 53.0225 64.77) (width 1.905) (layer "B.Cu") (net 2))
 (segment (start 48.26 60.0075) (end 38.1 60.0075) (width 1.905) (layer "B.Cu") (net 2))
 (segment (start 36.83 58.7375) (end 36.83 56.515) (width 1.905) (layer "B.Cu") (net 2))
 (segment (start 36.83 58.7375) (end 38.1 60.0075) (width 1.905) (layer "B.Cu") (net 2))
 (segment (start 46.6725 52.705) (end 42.8625 52.705) (width 1.905) (layer "B.Cu") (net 11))
 (segment (start 42.8625 52.705) (end 40.3225 50.165) (width 1.905) (layer "B.Cu") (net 11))
 (segment (start 40.3225 50.165) (end 39.0525 50.165) (width 1.905) (layer "B.Cu") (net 11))
 (segment (start 42.8625 55.245) (end 46.6725 55.245) (width 1.905) (layer "B.Cu") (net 12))
 (segment (start 39.0525 57.785) (end 40.3225 57.785) (width 1.905) (layer "B.Cu") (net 12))
 (segment (start 40.3225 57.785) (end 42.8625 55.245) (width 1.905) (layer "B.Cu") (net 12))
 (segment (start 62.23 45.72) (end 64.135 47.625) (width 1.905) (layer "B.Cu") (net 10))
 (segment (start 44.1325 50.165) (end 46.6725 50.165) (width 1.905) (layer "B.Cu") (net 10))
 (segment (start 64.135 47.625) (end 64.135 54.2925) (width 1.905) (layer "B.Cu") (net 10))
 (segment (start 64.135 54.2925) (end 68.8975 59.055) (width 1.905) (layer "B.Cu") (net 10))
 (segment (start 68.8975 76.835) (end 64.4525 81.28) (width 1.905) (layer "B.Cu") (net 10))
 (segment (start 46.6725 50.165) (end 51.1175 45.72) (width 1.905) (layer "B.Cu") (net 10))
 (segment (start 68.8975 59.055) (end 68.8975 76.835) (width 1.905) (layer "B.Cu") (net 10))
 (segment (start 51.1175 45.72) (end 62.23 45.72) (width 1.905) (layer "B.Cu") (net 10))
 (segment (start 56.832501 69.85) (end 54.2925 69.85) (width 1.905) (layer "B.Cu") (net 7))
 (segment (start 56.832501 69.85) (end 56.832501 72.350001) (width 1.905) (layer "B.Cu") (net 7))
 (segment (start 56.8325 81.28) (end 56.8325 79.375) (width 1.905) (layer "B.Cu") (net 9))
 (segment (start 56.8325 79.375) (end 61.9125 74.295) (width 1.905) (layer "B.Cu") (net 9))
 (segment (start 61.9125 74.295) (end 61.9125 72.39) (width 1.905) (layer "B.Cu") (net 9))
 (via (at 56.8325 55.245) (size 1.905) (drill 0.6) (layers "F.Cu" "B.Cu") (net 8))
 (via (at 61.9125 55.245) (size 1.905) (drill 0.6) (layers "F.Cu" "B.Cu") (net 8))
 (segment (start 54.2925 50.165) (end 56.8325 50.165) (width 1.905) (layer "B.Cu") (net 8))
 (segment (start 61.9125 80.645) (end 61.9125 81.28) (width 1.905) (layer "B.Cu") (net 8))
 (segment (start 54.2925 62.23) (end 51.7525 59.69) (width 1.905) (layer "B.Cu") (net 8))
 (segment (start 53.0225 50.165) (end 54.2925 50.165) (width 1.905) (layer "B.Cu") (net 8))
 (segment (start 56.8325 50.165) (end 56.8325 55.245) (width 1.905) (layer "B.Cu") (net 8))
 (segment (start 51.7525 51.435) (end 53.0225 50.165) (width 1.905) (layer "B.Cu") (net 8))
 (segment (start 61.9125 55.245) (end 66.675 60.0075) (width 1.905) (layer "B.Cu") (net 8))
 (segment (start 51.7525 59.69) (end 51.7525 51.435) (width 1.905) (layer "B.Cu") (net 8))
 (segment (start 56.8325 62.23) (end 54.2925 62.23) (width 1.905) (layer "B.Cu") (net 8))
 (segment (start 66.675 60.0075) (end 66.675 75.8825) (width 1.905) (layer "B.Cu") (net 8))
 (segment (start 66.675 75.8825) (end 61.9125 80.645) (width 1.905) (layer "B.Cu") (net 8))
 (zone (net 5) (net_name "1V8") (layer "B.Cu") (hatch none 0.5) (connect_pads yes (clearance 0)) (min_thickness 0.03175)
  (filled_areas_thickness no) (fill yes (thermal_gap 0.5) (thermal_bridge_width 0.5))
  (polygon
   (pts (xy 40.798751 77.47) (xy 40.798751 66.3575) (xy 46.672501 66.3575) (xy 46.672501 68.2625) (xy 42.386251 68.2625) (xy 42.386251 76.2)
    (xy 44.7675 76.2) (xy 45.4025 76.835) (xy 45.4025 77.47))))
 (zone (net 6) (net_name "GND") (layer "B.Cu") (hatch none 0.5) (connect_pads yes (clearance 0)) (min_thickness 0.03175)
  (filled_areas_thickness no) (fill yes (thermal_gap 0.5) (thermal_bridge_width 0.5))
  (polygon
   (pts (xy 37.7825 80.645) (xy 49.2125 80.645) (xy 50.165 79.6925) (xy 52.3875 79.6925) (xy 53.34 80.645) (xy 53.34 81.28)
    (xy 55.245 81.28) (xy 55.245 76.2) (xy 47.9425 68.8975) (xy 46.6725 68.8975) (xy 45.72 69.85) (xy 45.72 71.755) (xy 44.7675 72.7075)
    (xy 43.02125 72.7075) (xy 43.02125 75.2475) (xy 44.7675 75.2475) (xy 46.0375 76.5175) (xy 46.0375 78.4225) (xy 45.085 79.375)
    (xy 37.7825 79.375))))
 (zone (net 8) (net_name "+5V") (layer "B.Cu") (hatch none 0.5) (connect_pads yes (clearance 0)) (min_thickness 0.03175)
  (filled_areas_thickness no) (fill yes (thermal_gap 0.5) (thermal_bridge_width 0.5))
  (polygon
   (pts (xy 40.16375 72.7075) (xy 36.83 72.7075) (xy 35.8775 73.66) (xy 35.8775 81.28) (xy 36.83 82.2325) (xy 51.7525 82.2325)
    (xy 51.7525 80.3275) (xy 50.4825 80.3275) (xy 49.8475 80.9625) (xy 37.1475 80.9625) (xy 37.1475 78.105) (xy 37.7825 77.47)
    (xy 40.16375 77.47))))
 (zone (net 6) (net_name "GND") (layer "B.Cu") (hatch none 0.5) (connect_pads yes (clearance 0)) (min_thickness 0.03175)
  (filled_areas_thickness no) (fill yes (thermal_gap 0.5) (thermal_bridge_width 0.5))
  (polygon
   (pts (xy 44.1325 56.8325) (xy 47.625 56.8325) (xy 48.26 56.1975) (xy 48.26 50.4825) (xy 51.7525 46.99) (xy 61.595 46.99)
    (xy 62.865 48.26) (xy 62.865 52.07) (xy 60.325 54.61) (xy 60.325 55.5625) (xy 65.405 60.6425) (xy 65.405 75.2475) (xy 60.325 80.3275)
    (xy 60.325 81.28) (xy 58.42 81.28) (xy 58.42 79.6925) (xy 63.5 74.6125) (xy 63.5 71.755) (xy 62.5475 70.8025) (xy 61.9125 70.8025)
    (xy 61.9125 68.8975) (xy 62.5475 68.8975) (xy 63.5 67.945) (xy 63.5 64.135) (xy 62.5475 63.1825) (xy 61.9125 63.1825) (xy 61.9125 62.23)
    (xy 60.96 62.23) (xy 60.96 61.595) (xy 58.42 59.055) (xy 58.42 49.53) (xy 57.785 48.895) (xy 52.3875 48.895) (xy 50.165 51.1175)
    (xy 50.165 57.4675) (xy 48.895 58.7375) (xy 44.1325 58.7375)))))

